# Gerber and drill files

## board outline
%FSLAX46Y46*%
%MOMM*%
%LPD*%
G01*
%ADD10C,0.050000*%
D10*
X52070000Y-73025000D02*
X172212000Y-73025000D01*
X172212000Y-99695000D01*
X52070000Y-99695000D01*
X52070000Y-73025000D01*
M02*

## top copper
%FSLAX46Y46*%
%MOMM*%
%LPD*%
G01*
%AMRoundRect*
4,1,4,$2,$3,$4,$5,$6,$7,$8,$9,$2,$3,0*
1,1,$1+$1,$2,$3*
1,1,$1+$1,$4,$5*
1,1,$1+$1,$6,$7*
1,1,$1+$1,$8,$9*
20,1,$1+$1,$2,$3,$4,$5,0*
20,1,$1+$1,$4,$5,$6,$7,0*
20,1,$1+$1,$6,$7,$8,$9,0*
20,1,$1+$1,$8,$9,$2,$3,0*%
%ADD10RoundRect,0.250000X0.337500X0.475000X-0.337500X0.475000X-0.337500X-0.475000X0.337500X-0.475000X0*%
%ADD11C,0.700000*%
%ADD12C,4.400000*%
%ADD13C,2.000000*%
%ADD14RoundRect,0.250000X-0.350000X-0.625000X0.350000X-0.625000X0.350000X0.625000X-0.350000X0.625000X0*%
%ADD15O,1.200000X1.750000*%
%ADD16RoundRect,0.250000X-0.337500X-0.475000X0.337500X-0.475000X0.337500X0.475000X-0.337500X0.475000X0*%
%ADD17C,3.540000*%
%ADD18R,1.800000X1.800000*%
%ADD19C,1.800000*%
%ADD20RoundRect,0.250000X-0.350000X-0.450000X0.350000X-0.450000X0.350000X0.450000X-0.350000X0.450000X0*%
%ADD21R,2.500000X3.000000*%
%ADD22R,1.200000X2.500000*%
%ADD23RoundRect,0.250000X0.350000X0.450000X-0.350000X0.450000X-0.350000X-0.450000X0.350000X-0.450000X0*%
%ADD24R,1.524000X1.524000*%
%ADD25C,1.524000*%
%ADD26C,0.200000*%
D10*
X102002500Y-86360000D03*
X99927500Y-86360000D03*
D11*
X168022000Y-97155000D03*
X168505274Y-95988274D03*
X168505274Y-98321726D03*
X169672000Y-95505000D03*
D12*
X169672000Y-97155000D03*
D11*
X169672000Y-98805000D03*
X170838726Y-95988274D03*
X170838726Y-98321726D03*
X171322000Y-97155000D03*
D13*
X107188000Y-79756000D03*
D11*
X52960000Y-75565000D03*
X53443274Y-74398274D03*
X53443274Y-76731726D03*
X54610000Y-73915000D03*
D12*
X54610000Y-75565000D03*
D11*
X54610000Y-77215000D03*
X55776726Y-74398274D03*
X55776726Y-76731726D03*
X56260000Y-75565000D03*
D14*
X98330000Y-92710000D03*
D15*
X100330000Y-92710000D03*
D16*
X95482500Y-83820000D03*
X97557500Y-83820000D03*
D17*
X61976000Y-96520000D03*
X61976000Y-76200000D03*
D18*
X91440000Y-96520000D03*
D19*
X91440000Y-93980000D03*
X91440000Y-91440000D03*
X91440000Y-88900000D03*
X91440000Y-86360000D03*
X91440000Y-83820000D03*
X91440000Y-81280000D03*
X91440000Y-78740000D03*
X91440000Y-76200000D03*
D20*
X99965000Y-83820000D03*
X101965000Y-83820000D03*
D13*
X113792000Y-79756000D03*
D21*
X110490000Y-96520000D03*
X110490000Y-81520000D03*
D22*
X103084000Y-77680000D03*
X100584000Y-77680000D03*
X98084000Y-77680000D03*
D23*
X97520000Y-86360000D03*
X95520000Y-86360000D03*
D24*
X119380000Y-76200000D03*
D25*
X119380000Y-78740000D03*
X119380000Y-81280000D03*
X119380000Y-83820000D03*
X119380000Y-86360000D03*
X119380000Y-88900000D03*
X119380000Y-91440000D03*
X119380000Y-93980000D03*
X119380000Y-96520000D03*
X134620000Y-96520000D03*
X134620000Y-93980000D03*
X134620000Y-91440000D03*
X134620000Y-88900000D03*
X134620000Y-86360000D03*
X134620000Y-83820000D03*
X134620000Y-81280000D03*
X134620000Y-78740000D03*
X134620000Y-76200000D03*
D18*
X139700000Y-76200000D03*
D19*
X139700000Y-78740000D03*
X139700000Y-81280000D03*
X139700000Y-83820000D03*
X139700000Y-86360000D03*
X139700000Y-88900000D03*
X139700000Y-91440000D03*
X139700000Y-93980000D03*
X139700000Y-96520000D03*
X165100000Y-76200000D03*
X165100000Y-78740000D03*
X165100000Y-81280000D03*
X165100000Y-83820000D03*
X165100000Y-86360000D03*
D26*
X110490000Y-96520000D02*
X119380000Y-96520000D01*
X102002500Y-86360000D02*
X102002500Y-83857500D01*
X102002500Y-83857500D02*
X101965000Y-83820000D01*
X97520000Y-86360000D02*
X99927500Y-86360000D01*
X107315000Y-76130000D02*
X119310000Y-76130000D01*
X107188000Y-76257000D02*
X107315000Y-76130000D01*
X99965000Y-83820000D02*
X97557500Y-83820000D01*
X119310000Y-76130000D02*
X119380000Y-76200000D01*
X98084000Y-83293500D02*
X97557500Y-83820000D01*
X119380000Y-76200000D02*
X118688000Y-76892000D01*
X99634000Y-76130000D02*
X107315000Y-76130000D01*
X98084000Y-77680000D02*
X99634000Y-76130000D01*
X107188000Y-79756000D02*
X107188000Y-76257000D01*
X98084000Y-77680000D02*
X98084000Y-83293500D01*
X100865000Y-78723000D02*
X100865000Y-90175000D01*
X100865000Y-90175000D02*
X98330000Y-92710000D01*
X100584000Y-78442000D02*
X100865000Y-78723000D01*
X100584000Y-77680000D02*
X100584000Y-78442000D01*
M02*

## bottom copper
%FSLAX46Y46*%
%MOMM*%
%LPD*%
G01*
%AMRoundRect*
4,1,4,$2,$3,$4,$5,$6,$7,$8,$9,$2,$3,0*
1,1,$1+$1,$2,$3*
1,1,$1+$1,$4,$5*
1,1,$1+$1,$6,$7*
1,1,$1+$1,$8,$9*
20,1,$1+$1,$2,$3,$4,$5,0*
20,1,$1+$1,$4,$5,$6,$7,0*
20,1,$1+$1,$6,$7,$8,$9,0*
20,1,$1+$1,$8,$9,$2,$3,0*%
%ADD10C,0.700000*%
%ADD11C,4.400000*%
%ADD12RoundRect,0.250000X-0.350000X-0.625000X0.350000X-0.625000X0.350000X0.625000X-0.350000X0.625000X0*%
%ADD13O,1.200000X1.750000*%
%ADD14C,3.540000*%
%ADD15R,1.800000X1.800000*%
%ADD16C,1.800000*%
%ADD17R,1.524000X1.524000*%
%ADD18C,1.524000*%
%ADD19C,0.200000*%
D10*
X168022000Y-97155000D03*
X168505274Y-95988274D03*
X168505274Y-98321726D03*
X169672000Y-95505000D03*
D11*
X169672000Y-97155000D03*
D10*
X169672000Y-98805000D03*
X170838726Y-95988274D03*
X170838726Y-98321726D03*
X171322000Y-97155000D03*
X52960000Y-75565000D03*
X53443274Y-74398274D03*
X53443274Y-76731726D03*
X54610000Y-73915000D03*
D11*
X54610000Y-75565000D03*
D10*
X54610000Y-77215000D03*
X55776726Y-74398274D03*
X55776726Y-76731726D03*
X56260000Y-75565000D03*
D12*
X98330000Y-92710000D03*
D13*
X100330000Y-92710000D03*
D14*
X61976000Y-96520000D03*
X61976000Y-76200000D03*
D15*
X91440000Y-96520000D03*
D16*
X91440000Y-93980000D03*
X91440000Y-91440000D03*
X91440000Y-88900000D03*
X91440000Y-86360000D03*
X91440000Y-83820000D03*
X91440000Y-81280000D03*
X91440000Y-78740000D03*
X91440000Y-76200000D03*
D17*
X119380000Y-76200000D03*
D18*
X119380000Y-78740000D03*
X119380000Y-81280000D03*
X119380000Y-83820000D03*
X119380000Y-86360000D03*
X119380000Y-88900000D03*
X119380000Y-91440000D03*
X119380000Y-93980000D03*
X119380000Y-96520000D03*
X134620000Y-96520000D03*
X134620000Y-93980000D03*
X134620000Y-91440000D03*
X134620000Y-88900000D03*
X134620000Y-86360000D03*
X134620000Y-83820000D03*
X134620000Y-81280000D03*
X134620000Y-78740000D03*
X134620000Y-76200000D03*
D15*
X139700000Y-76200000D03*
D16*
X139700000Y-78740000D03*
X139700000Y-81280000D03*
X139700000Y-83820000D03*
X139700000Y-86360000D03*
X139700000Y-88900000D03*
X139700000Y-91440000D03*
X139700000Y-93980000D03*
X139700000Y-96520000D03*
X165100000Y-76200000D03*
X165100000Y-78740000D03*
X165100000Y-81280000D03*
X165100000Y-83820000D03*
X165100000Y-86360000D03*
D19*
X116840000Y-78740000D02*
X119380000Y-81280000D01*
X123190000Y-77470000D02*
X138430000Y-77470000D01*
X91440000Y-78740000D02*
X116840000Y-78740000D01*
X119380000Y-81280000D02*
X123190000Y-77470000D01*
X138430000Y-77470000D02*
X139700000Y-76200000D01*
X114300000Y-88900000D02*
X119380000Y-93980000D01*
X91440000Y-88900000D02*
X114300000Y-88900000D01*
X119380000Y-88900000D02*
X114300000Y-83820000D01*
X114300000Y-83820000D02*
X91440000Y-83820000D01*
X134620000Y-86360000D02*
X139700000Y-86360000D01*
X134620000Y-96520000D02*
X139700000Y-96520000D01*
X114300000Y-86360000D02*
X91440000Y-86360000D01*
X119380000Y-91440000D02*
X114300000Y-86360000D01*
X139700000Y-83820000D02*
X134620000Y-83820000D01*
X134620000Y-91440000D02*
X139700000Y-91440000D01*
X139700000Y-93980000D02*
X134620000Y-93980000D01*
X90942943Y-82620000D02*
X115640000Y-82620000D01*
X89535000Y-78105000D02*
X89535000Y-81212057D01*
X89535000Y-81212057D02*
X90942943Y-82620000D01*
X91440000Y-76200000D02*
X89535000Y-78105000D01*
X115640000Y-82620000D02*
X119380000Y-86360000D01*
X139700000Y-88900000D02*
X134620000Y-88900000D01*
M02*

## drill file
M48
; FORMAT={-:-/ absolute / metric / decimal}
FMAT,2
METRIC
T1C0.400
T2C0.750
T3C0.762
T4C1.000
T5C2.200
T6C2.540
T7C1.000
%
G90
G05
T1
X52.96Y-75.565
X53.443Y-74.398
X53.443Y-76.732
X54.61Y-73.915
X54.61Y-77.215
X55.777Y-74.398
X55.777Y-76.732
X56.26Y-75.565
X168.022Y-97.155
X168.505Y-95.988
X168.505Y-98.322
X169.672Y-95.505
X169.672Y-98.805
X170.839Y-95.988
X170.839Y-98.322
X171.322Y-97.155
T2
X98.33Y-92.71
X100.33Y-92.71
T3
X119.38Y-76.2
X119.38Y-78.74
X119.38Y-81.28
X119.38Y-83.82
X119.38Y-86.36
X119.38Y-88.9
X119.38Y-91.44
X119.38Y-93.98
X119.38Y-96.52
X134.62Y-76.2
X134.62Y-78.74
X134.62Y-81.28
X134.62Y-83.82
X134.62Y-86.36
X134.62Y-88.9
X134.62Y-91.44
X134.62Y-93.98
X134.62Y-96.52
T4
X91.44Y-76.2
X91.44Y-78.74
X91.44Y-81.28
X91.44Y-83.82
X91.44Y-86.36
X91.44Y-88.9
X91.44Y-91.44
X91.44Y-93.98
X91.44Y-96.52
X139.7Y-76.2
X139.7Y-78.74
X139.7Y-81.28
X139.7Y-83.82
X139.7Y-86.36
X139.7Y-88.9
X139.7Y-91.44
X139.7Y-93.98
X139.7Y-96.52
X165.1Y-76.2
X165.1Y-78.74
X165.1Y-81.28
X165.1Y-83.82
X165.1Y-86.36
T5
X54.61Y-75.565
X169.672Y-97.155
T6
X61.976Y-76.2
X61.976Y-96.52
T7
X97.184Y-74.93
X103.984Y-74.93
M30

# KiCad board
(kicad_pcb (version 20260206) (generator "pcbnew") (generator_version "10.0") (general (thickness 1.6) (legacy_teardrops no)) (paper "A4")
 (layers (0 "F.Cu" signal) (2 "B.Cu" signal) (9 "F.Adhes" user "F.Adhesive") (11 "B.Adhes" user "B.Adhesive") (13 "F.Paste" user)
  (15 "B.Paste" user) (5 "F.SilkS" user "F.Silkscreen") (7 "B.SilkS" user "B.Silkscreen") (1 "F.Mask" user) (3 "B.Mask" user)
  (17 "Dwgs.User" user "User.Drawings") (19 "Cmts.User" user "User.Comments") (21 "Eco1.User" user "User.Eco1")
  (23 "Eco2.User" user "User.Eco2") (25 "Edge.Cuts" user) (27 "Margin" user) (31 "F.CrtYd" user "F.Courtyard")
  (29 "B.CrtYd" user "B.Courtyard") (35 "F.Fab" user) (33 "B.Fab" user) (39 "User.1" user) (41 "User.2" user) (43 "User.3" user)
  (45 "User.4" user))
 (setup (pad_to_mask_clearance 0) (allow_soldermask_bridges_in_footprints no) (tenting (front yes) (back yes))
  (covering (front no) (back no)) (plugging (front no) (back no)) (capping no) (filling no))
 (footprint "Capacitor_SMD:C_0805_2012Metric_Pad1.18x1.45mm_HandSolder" (layer "F.Cu") (at 100.965 86.36 180)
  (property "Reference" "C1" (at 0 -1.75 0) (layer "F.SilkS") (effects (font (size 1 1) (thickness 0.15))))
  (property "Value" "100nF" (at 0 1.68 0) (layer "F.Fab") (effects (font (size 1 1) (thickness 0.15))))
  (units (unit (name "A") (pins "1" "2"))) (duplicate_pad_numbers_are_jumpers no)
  (pad "1" smd roundrect (at -1.0375 0 180) (size 1.175 1.45) (layers "F.Cu" "F.Mask" "F.Paste") (roundrect_rratio 0.212766)
   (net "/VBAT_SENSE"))
  (pad "2" smd roundrect (at 1.0375 0 180) (size 1.175 1.45) (layers "F.Cu" "F.Mask" "F.Paste") (roundrect_rratio 0.212766)
   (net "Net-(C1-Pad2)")))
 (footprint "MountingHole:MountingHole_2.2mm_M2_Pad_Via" (layer "F.Cu") (at 169.672 97.155)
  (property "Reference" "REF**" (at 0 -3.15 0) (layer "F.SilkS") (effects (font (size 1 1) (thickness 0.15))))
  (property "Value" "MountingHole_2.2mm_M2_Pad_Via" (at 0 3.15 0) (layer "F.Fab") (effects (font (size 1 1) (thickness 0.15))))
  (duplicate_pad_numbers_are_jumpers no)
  (pad "1" thru_hole circle (at -1.65 0) (size 0.7 0.7) (drill 0.4) (layers "*.Cu" "*.Mask") (remove_unused_layers no) (zone_connect 2))
  (pad "1" thru_hole circle (at -1.166726 -1.166726) (size 0.7 0.7) (drill 0.4) (layers "*.Cu" "*.Mask") (remove_unused_layers no)
   (zone_connect 2))
  (pad "1" thru_hole circle (at -1.166726 1.166726) (size 0.7 0.7) (drill 0.4) (layers "*.Cu" "*.Mask") (remove_unused_layers no)
   (zone_connect 2))
  (pad "1" thru_hole circle (at 0 -1.65) (size 0.7 0.7) (drill 0.4) (layers "*.Cu" "*.Mask") (remove_unused_layers no) (zone_connect 2))
  (pad "1" thru_hole circle (at 0 0) (size 4.4 4.4) (drill 2.2) (layers "*.Cu" "*.Mask") (remove_unused_layers no) (zone_connect 2))
  (pad "1" thru_hole circle (at 0 1.65) (size 0.7 0.7) (drill 0.4) (layers "*.Cu" "*.Mask") (remove_unused_layers no) (zone_connect 2))
  (pad "1" thru_hole circle (at 1.166726 -1.166726) (size 0.7 0.7) (drill 0.4) (layers "*.Cu" "*.Mask") (remove_unused_layers no)
   (zone_connect 2))
  (pad "1" thru_hole circle (at 1.166726 1.166726) (size 0.7 0.7) (drill 0.4) (layers "*.Cu" "*.Mask") (remove_unused_layers no)
   (zone_connect 2))
  (pad "1" thru_hole circle (at 1.65 0) (size 0.7 0.7) (drill 0.4) (layers "*.Cu" "*.Mask") (remove_unused_layers no) (zone_connect 2)))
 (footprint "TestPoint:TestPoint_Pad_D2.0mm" (layer "F.Cu") (at 107.188 79.756 180)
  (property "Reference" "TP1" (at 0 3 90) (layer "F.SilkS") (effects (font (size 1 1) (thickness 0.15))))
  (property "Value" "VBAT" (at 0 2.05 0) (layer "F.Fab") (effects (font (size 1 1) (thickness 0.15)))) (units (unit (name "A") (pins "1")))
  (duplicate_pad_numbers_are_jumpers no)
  (pad "1" smd circle (at 0 0 180) (size 2 2) (layers "F.Cu" "F.Mask") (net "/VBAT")))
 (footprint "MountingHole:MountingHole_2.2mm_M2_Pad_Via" (layer "F.Cu") (at 54.61 75.565)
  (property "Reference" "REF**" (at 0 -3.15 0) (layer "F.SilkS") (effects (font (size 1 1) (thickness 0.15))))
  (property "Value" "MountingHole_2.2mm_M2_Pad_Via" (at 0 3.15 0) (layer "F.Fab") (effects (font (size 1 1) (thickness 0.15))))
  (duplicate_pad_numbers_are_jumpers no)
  (pad "1" thru_hole circle (at -1.65 0) (size 0.7 0.7) (drill 0.4) (layers "*.Cu" "*.Mask") (remove_unused_layers no) (zone_connect 2))
  (pad "1" thru_hole circle (at -1.166726 -1.166726) (size 0.7 0.7) (drill 0.4) (layers "*.Cu" "*.Mask") (remove_unused_layers no)
   (zone_connect 2))
  (pad "1" thru_hole circle (at -1.166726 1.166726) (size 0.7 0.7) (drill 0.4) (layers "*.Cu" "*.Mask") (remove_unused_layers no)
   (zone_connect 2))
  (pad "1" thru_hole circle (at 0 -1.65) (size 0.7 0.7) (drill 0.4) (layers "*.Cu" "*.Mask") (remove_unused_layers no) (zone_connect 2))
  (pad "1" thru_hole circle (at 0 0) (size 4.4 4.4) (drill 2.2) (layers "*.Cu" "*.Mask") (remove_unused_layers no) (zone_connect 2))
  (pad "1" thru_hole circle (at 0 1.65) (size 0.7 0.7) (drill 0.4) (layers "*.Cu" "*.Mask") (remove_unused_layers no) (zone_connect 2))
  (pad "1" thru_hole circle (at 1.166726 -1.166726) (size 0.7 0.7) (drill 0.4) (layers "*.Cu" "*.Mask") (remove_unused_layers no)
   (zone_connect 2))
  (pad "1" thru_hole circle (at 1.166726 1.166726) (size 0.7 0.7) (drill 0.4) (layers "*.Cu" "*.Mask") (remove_unused_layers no)
   (zone_connect 2))
  (pad "1" thru_hole circle (at 1.65 0) (size 0.7 0.7) (drill 0.4) (layers "*.Cu" "*.Mask") (remove_unused_layers no) (zone_connect 2)))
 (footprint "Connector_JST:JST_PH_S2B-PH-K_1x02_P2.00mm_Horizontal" (layer "F.Cu") (at 98.33 92.71)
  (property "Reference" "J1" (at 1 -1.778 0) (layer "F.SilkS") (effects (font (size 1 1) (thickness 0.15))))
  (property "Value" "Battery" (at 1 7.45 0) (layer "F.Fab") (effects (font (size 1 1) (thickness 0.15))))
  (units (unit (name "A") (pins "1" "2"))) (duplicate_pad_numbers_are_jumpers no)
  (pad "1" thru_hole roundrect (at 0 0) (size 1.2 1.75) (drill 0.75) (layers "*.Cu" "*.Mask") (remove_unused_layers no)
   (roundrect_rratio 0.208333) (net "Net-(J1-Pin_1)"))
  (pad "2" thru_hole oval (at 2 0) (size 1.2 1.75) (drill 0.75) (layers "*.Cu" "*.Mask") (remove_unused_layers no) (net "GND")))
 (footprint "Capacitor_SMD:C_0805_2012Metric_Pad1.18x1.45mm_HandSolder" (layer "F.Cu") (at 96.52 83.82)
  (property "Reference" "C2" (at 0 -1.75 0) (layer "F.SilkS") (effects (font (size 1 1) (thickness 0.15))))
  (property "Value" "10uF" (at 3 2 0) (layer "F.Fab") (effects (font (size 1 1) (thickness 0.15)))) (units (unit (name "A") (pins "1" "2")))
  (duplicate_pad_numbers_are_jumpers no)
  (pad "1" smd roundrect (at -1.0375 0) (size 1.175 1.45) (layers "F.Cu" "F.Mask" "F.Paste") (roundrect_rratio 0.212766) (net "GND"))
  (pad "2" smd roundrect (at 1.0375 0) (size 1.175 1.45) (layers "F.Cu" "F.Mask" "F.Paste") (roundrect_rratio 0.212766) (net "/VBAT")))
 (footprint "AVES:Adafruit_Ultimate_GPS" (layer "F.Cu") (at 91.44 96.52 90)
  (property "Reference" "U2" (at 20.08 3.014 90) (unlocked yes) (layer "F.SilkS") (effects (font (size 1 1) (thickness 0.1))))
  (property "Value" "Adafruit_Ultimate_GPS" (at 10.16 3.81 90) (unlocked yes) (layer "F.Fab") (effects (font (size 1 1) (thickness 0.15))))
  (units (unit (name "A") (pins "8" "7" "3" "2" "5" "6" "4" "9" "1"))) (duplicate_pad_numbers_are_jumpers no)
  (pad "" thru_hole circle (at 0 -29.464 90) (size 3.54 3.54) (drill 2.54) (layers "*.Cu" "*.Mask") (remove_unused_layers no))
  (pad "" thru_hole circle (at 20.32 -29.464 90) (size 3.54 3.54) (drill 2.54) (layers "*.Cu" "*.Mask") (remove_unused_layers no))
  (pad "1" thru_hole rect (at 0 0 90) (size 1.8 1.8) (drill 1) (layers "*.Cu" "*.Mask") (remove_unused_layers no)
   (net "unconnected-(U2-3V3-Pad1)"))
  (pad "2" thru_hole circle (at 2.54 0 90) (size 1.8 1.8) (drill 1) (layers "*.Cu" "*.Mask") (remove_unused_layers no)
   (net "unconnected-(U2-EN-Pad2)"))
  (pad "3" thru_hole circle (at 5.08 0 90) (size 1.8 1.8) (drill 1) (layers "*.Cu" "*.Mask") (remove_unused_layers no)
   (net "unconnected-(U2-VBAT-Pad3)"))
  (pad "4" thru_hole circle (at 7.62 0 90) (size 1.8 1.8) (drill 1) (layers "*.Cu" "*.Mask") (remove_unused_layers no) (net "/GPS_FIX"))
  (pad "5" thru_hole circle (at 10.16 0 90) (size 1.8 1.8) (drill 1) (layers "*.Cu" "*.Mask") (remove_unused_layers no) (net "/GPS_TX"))
  (pad "6" thru_hole circle (at 12.7 0 90) (size 1.8 1.8) (drill 1) (layers "*.Cu" "*.Mask") (remove_unused_layers no) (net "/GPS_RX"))
  (pad "7" thru_hole circle (at 15.24 0 90) (size 1.8 1.8) (drill 1) (layers "*.Cu" "*.Mask") (remove_unused_layers no) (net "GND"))
  (pad "8" thru_hole circle (at 17.78 0 90) (size 1.8 1.8) (drill 1) (layers "*.Cu" "*.Mask") (remove_unused_layers no) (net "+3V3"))
  (pad "9" thru_hole circle (at 20.32 0 90) (size 1.8 1.8) (drill 1) (layers "*.Cu" "*.Mask") (remove_unused_layers no) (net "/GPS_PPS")))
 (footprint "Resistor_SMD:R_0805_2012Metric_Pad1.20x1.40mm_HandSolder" (layer "F.Cu") (at 100.965 83.82)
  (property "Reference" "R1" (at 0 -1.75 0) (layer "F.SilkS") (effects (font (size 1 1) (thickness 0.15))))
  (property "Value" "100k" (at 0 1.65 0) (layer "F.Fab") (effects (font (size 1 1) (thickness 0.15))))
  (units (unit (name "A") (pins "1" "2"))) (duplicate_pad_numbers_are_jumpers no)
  (pad "1" smd roundrect (at -1 0) (size 1.2 1.4) (layers "F.Cu" "F.Mask" "F.Paste") (roundrect_rratio 0.208333) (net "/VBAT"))
  (pad "2" smd roundrect (at 1 0) (size 1.2 1.4) (layers "F.Cu" "F.Mask" "F.Paste") (roundrect_rratio 0.208333) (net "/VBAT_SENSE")))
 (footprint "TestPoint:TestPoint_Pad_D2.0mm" (layer "F.Cu") (at 113.792 79.756 180)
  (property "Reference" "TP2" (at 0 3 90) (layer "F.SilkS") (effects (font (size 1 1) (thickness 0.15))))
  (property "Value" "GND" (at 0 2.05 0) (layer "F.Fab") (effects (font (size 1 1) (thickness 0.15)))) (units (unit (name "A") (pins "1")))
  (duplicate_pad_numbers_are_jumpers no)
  (pad "1" smd circle (at 0 0 180) (size 2 2) (layers "F.Cu" "F.Mask") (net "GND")))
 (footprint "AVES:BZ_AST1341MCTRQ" (layer "F.Cu") (at 116.99 95.52 90)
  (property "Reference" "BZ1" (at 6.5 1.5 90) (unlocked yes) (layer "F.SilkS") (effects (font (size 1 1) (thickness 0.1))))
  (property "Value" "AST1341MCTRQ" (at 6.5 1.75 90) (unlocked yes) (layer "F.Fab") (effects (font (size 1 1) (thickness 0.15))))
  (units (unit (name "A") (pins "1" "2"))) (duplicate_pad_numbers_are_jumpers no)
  (pad "1" smd rect (at -1 -6.5 180) (size 2.5 3) (layers "F.Cu" "F.Mask" "F.Paste") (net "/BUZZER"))
  (pad "2" smd rect (at 14 -6.5 180) (size 2.5 3) (layers "F.Cu" "F.Mask" "F.Paste") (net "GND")))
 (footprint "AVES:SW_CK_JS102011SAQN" (layer "F.Cu") (at 100.584 74.93 180)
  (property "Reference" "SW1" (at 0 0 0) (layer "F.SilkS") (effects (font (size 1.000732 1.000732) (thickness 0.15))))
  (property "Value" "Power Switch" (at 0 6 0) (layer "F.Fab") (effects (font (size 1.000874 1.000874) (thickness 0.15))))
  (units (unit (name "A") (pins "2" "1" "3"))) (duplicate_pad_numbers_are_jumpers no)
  (pad "" np_thru_hole circle (at -3.4 0 180) (size 1 1) (drill 1) (layers "*.Cu" "*.Mask"))
  (pad "" np_thru_hole circle (at 3.4 0 180) (size 1 1) (drill 1) (layers "*.Cu" "*.Mask"))
  (pad "1" smd rect (at -2.5 -2.75 180) (size 1.2 2.5) (layers "F.Cu" "F.Mask" "F.Paste") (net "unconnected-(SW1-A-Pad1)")
   (solder_mask_margin 0.102))
  (pad "2" smd rect (at 0 -2.75 180) (size 1.2 2.5) (layers "F.Cu" "F.Mask" "F.Paste") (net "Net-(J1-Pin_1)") (solder_mask_margin 0.102))
  (pad "3" smd rect (at 2.5 -2.75 180) (size 1.2 2.5) (layers "F.Cu" "F.Mask" "F.Paste") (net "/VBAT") (solder_mask_margin 0.102)))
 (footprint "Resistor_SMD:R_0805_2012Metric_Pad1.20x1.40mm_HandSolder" (layer "F.Cu") (at 96.52 86.36 180)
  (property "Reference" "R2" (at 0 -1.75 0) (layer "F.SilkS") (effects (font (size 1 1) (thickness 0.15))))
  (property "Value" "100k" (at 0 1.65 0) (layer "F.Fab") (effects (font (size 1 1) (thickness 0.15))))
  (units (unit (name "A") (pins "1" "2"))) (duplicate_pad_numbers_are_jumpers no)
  (pad "1" smd roundrect (at -1 0 180) (size 1.2 1.4) (layers "F.Cu" "F.Mask" "F.Paste") (roundrect_rratio 0.208333) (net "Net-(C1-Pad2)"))
  (pad "2" smd roundrect (at 1 0 180) (size 1.2 1.4) (layers "F.Cu" "F.Mask" "F.Paste") (roundrect_rratio 0.208333) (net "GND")))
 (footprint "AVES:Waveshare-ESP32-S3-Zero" (layer "F.Cu") (at 118 74.61)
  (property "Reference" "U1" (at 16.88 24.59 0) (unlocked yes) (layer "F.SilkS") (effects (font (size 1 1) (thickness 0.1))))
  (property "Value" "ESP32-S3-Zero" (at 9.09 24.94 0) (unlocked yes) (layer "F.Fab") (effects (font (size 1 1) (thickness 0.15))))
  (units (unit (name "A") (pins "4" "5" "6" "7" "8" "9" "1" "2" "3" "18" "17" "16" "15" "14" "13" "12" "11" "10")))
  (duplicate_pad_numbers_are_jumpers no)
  (pad "1" thru_hole rect (at 1.38 1.59) (size 1.524 1.524) (drill 0.762) (layers "*.Cu" "*.Mask") (remove_unused_layers no) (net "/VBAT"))
  (pad "2" thru_hole circle (at 1.38 4.13) (size 1.524 1.524) (drill 0.762) (layers "*.Cu" "*.Mask") (remove_unused_layers no) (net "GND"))
  (pad "3" thru_hole circle (at 1.38 6.67) (size 1.524 1.524) (drill 0.762) (layers "*.Cu" "*.Mask") (remove_unused_layers no) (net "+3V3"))
  (pad "4" thru_hole circle (at 1.38 9.21) (size 1.524 1.524) (drill 0.762) (layers "*.Cu" "*.Mask") (remove_unused_layers no)
   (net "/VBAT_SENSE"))
  (pad "5" thru_hole circle (at 1.38 11.75) (size 1.524 1.524) (drill 0.762) (layers "*.Cu" "*.Mask") (remove_unused_layers no)
   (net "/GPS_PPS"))
  (pad "6" thru_hole circle (at 1.38 14.29) (size 1.524 1.524) (drill 0.762) (layers "*.Cu" "*.Mask") (remove_unused_layers no)
   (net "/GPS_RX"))
  (pad "7" thru_hole circle (at 1.38 16.83) (size 1.524 1.524) (drill 0.762) (layers "*.Cu" "*.Mask") (remove_unused_layers no)
   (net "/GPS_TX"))
  (pad "8" thru_hole circle (at 1.38 19.37) (size 1.524 1.524) (drill 0.762) (layers "*.Cu" "*.Mask") (remove_unused_layers no)
   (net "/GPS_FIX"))
  (pad "9" thru_hole circle (at 1.38 21.91) (size 1.524 1.524) (drill 0.762) (layers "*.Cu" "*.Mask") (remove_unused_layers no)
   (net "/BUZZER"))
  (pad "10" thru_hole circle (at 16.62 21.91) (size 1.524 1.524) (drill 0.762) (layers "*.Cu" "*.Mask") (remove_unused_layers no)
   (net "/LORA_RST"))
  (pad "11" thru_hole circle (at 16.62 19.37) (size 1.524 1.524) (drill 0.762) (layers "*.Cu" "*.Mask") (remove_unused_layers no)
   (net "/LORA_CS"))
  (pad "12" thru_hole circle (at 16.62 16.83) (size 1.524 1.524) (drill 0.762) (layers "*.Cu" "*.Mask") (remove_unused_layers no)
   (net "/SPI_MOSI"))
  (pad "13" thru_hole circle (at 16.62 14.29) (size 1.524 1.524) (drill 0.762) (layers "*.Cu" "*.Mask") (remove_unused_layers no)
   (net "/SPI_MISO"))
  (pad "14" thru_hole circle (at 16.62 11.75) (size 1.524 1.524) (drill 0.762) (layers "*.Cu" "*.Mask") (remove_unused_layers no)
   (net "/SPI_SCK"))
  (pad "15" thru_hole circle (at 16.62 9.21) (size 1.524 1.524) (drill 0.762) (layers "*.Cu" "*.Mask") (remove_unused_layers no)
   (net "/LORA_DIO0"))
  (pad "16" thru_hole circle (at 16.62 6.67) (size 1.524 1.524) (drill 0.762) (layers "*.Cu" "*.Mask") (remove_unused_layers no)
   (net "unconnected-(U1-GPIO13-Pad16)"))
  (pad "17" thru_hole circle (at 16.62 4.13) (size 1.524 1.524) (drill 0.762) (layers "*.Cu" "*.Mask") (remove_unused_layers no)
   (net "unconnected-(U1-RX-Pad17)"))
  (pad "18" thru_hole circle (at 16.62 1.59) (size 1.524 1.524) (drill 0.762) (layers "*.Cu" "*.Mask") (remove_unused_layers no)
   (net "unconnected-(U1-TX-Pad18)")))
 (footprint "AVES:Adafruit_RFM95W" (layer "F.Cu") (at 139.7 76.2 -90)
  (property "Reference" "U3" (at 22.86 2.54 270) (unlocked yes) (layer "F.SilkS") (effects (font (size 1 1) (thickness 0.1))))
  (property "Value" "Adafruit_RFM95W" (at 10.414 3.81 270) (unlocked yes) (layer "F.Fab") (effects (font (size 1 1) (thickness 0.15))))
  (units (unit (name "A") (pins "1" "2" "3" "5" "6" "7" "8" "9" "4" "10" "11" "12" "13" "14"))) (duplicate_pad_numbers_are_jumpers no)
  (pad "1" thru_hole rect (at 0 0 270) (size 1.8 1.8) (drill 1) (layers "*.Cu" "*.Mask") (remove_unused_layers no) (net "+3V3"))
  (pad "2" thru_hole circle (at 2.54 0 270) (size 1.8 1.8) (drill 1) (layers "*.Cu" "*.Mask") (remove_unused_layers no) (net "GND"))
  (pad "3" thru_hole circle (at 5.08 0 270) (size 1.8 1.8) (drill 1) (layers "*.Cu" "*.Mask") (remove_unused_layers no)
   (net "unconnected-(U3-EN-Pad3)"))
  (pad "4" thru_hole circle (at 7.62 0 270) (size 1.8 1.8) (drill 1) (layers "*.Cu" "*.Mask") (remove_unused_layers no) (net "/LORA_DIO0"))
  (pad "5" thru_hole circle (at 10.16 0 270) (size 1.8 1.8) (drill 1) (layers "*.Cu" "*.Mask") (remove_unused_layers no) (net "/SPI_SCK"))
  (pad "6" thru_hole circle (at 12.7 0 270) (size 1.8 1.8) (drill 1) (layers "*.Cu" "*.Mask") (remove_unused_layers no) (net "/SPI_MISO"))
  (pad "7" thru_hole circle (at 15.24 0 270) (size 1.8 1.8) (drill 1) (layers "*.Cu" "*.Mask") (remove_unused_layers no) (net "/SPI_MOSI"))
  (pad "8" thru_hole circle (at 17.78 0 270) (size 1.8 1.8) (drill 1) (layers "*.Cu" "*.Mask") (remove_unused_layers no) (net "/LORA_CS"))
  (pad "9" thru_hole circle (at 20.32 0 270) (size 1.8 1.8) (drill 1) (layers "*.Cu" "*.Mask") (remove_unused_layers no) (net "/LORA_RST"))
  (pad "10" thru_hole circle (at 0 -25.4 270) (size 1.8 1.8) (drill 1) (layers "*.Cu" "*.Mask") (remove_unused_layers no)
   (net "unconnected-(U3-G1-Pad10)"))
  (pad "11" thru_hole circle (at 2.54 -25.4 270) (size 1.8 1.8) (drill 1) (layers "*.Cu" "*.Mask") (remove_unused_layers no)
   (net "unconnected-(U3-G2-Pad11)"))
  (pad "12" thru_hole circle (at 5.08 -25.4 270) (size 1.8 1.8) (drill 1) (layers "*.Cu" "*.Mask") (remove_unused_layers no)
   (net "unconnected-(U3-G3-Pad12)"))
  (pad "13" thru_hole circle (at 7.62 -25.4 270) (size 1.8 1.8) (drill 1) (layers "*.Cu" "*.Mask") (remove_unused_layers no)
   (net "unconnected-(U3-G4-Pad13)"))
  (pad "14" thru_hole circle (at 10.16 -25.4 270) (size 1.8 1.8) (drill 1) (layers "*.Cu" "*.Mask") (remove_unused_layers no)
   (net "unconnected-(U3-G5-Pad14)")))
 (gr_rect (start 52.07 73.025) (end 172.212 99.695) (stroke (width 0.05) (type default)) (fill no) (layer "Edge.Cuts"))
 (segment (start 110.49 96.52) (end 119.38 96.52) (width 0.2) (layer "F.Cu") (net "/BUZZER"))
 (segment (start 102.0025 86.36) (end 102.0025 83.8575) (width 0.2) (layer "F.Cu") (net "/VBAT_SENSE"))
 (segment (start 102.0025 83.8575) (end 101.965 83.82) (width 0.2) (layer "F.Cu") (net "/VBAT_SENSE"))
 (segment (start 97.52 86.36) (end 99.9275 86.36) (width 0.2) (layer "F.Cu") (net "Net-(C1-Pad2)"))
 (segment (start 107.315 76.13) (end 119.31 76.13) (width 0.2) (layer "F.Cu") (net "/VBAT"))
 (segment (start 107.188 76.257) (end 107.315 76.13) (width 0.2) (layer "F.Cu") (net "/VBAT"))
 (segment (start 99.965 83.82) (end 97.5575 83.82) (width 0.2) (layer "F.Cu") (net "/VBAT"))
 (segment (start 119.31 76.13) (end 119.38 76.2) (width 0.2) (layer "F.Cu") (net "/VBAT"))
 (segment (start 98.084 83.2935) (end 97.5575 83.82) (width 0.2) (layer "F.Cu") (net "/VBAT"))
 (segment (start 119.38 76.2) (end 118.688 76.892) (width 0.2) (layer "F.Cu") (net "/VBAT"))
 (segment (start 99.634 76.13) (end 107.315 76.13) (width 0.2) (layer "F.Cu") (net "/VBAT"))
 (segment (start 98.084 77.68) (end 99.634 76.13) (width 0.2) (layer "F.Cu") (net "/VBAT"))
 (segment (start 107.188 79.756) (end 107.188 76.257) (width 0.2) (layer "F.Cu") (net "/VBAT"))
 (segment (start 98.084 77.68) (end 98.084 83.2935) (width 0.2) (layer "F.Cu") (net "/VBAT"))
 (segment (start 100.865 78.723) (end 100.865 90.175) (width 0.2) (layer "F.Cu") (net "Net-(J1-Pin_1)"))
 (segment (start 100.865 90.175) (end 98.33 92.71) (width 0.2) (layer "F.Cu") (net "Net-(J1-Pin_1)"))
 (segment (start 100.584 78.442) (end 100.865 78.723) (width 0.2) (layer "F.Cu") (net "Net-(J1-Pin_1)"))
 (segment (start 100.584 77.68) (end 100.584 78.442) (width 0.2) (layer "F.Cu") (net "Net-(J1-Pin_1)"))
 (segment (start 116.84 78.74) (end 119.38 81.28) (width 0.2) (layer "B.Cu") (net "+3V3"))
 (segment (start 123.19 77.47) (end 138.43 77.47) (width 0.2) (layer "B.Cu") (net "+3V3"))
 (segment (start 91.44 78.74) (end 116.84 78.74) (width 0.2) (layer "B.Cu") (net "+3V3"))
 (segment (start 119.38 81.28) (end 123.19 77.47) (width 0.2) (layer "B.Cu") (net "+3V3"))
 (segment (start 138.43 77.47) (end 139.7 76.2) (width 0.2) (layer "B.Cu") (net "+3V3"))
 (segment (start 114.3 88.9) (end 119.38 93.98) (width 0.2) (layer "B.Cu") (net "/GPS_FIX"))
 (segment (start 91.44 88.9) (end 114.3 88.9) (width 0.2) (layer "B.Cu") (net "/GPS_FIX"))
 (segment (start 119.38 88.9) (end 114.3 83.82) (width 0.2) (layer "B.Cu") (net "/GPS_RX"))
 (segment (start 114.3 83.82) (end 91.44 83.82) (width 0.2) (layer "B.Cu") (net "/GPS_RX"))
 (segment (start 134.62 86.36) (end 139.7 86.36) (width 0.2) (layer "B.Cu") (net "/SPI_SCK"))
 (segment (start 134.62 96.52) (end 139.7 96.52) (width 0.2) (layer "B.Cu") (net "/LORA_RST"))
 (segment (start 114.3 86.36) (end 91.44 86.36) (width 0.2) (layer "B.Cu") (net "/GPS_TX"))
 (segment (start 119.38 91.44) (end 114.3 86.36) (width 0.2) (layer "B.Cu") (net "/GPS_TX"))
 (segment (start 139.7 83.82) (end 134.62 83.82) (width 0.2) (layer "B.Cu") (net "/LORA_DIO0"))
 (segment (start 134.62 91.44) (end 139.7 91.44) (width 0.2) (layer "B.Cu") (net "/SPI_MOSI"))
 (segment (start 139.7 93.98) (end 134.62 93.98) (width 0.2) (layer "B.Cu") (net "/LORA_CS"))
 (segment (start 90.942943 82.62) (end 115.64 82.62) (width 0.2) (layer "B.Cu") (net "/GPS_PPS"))
 (segment (start 89.535 78.105) (end 89.535 81.212057) (width 0.2) (layer "B.Cu") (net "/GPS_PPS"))
 (segment (start 89.535 81.212057) (end 90.942943 82.62) (width 0.2) (layer "B.Cu") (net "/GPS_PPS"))
 (segment (start 91.44 76.2) (end 89.535 78.105) (width 0.2) (layer "B.Cu") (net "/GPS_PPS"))
 (segment (start 115.64 82.62) (end 119.38 86.36) (width 0.2) (layer "B.Cu") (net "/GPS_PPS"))
 (segment (start 139.7 88.9) (end 134.62 88.9) (width 0.2) (layer "B.Cu") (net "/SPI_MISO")))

